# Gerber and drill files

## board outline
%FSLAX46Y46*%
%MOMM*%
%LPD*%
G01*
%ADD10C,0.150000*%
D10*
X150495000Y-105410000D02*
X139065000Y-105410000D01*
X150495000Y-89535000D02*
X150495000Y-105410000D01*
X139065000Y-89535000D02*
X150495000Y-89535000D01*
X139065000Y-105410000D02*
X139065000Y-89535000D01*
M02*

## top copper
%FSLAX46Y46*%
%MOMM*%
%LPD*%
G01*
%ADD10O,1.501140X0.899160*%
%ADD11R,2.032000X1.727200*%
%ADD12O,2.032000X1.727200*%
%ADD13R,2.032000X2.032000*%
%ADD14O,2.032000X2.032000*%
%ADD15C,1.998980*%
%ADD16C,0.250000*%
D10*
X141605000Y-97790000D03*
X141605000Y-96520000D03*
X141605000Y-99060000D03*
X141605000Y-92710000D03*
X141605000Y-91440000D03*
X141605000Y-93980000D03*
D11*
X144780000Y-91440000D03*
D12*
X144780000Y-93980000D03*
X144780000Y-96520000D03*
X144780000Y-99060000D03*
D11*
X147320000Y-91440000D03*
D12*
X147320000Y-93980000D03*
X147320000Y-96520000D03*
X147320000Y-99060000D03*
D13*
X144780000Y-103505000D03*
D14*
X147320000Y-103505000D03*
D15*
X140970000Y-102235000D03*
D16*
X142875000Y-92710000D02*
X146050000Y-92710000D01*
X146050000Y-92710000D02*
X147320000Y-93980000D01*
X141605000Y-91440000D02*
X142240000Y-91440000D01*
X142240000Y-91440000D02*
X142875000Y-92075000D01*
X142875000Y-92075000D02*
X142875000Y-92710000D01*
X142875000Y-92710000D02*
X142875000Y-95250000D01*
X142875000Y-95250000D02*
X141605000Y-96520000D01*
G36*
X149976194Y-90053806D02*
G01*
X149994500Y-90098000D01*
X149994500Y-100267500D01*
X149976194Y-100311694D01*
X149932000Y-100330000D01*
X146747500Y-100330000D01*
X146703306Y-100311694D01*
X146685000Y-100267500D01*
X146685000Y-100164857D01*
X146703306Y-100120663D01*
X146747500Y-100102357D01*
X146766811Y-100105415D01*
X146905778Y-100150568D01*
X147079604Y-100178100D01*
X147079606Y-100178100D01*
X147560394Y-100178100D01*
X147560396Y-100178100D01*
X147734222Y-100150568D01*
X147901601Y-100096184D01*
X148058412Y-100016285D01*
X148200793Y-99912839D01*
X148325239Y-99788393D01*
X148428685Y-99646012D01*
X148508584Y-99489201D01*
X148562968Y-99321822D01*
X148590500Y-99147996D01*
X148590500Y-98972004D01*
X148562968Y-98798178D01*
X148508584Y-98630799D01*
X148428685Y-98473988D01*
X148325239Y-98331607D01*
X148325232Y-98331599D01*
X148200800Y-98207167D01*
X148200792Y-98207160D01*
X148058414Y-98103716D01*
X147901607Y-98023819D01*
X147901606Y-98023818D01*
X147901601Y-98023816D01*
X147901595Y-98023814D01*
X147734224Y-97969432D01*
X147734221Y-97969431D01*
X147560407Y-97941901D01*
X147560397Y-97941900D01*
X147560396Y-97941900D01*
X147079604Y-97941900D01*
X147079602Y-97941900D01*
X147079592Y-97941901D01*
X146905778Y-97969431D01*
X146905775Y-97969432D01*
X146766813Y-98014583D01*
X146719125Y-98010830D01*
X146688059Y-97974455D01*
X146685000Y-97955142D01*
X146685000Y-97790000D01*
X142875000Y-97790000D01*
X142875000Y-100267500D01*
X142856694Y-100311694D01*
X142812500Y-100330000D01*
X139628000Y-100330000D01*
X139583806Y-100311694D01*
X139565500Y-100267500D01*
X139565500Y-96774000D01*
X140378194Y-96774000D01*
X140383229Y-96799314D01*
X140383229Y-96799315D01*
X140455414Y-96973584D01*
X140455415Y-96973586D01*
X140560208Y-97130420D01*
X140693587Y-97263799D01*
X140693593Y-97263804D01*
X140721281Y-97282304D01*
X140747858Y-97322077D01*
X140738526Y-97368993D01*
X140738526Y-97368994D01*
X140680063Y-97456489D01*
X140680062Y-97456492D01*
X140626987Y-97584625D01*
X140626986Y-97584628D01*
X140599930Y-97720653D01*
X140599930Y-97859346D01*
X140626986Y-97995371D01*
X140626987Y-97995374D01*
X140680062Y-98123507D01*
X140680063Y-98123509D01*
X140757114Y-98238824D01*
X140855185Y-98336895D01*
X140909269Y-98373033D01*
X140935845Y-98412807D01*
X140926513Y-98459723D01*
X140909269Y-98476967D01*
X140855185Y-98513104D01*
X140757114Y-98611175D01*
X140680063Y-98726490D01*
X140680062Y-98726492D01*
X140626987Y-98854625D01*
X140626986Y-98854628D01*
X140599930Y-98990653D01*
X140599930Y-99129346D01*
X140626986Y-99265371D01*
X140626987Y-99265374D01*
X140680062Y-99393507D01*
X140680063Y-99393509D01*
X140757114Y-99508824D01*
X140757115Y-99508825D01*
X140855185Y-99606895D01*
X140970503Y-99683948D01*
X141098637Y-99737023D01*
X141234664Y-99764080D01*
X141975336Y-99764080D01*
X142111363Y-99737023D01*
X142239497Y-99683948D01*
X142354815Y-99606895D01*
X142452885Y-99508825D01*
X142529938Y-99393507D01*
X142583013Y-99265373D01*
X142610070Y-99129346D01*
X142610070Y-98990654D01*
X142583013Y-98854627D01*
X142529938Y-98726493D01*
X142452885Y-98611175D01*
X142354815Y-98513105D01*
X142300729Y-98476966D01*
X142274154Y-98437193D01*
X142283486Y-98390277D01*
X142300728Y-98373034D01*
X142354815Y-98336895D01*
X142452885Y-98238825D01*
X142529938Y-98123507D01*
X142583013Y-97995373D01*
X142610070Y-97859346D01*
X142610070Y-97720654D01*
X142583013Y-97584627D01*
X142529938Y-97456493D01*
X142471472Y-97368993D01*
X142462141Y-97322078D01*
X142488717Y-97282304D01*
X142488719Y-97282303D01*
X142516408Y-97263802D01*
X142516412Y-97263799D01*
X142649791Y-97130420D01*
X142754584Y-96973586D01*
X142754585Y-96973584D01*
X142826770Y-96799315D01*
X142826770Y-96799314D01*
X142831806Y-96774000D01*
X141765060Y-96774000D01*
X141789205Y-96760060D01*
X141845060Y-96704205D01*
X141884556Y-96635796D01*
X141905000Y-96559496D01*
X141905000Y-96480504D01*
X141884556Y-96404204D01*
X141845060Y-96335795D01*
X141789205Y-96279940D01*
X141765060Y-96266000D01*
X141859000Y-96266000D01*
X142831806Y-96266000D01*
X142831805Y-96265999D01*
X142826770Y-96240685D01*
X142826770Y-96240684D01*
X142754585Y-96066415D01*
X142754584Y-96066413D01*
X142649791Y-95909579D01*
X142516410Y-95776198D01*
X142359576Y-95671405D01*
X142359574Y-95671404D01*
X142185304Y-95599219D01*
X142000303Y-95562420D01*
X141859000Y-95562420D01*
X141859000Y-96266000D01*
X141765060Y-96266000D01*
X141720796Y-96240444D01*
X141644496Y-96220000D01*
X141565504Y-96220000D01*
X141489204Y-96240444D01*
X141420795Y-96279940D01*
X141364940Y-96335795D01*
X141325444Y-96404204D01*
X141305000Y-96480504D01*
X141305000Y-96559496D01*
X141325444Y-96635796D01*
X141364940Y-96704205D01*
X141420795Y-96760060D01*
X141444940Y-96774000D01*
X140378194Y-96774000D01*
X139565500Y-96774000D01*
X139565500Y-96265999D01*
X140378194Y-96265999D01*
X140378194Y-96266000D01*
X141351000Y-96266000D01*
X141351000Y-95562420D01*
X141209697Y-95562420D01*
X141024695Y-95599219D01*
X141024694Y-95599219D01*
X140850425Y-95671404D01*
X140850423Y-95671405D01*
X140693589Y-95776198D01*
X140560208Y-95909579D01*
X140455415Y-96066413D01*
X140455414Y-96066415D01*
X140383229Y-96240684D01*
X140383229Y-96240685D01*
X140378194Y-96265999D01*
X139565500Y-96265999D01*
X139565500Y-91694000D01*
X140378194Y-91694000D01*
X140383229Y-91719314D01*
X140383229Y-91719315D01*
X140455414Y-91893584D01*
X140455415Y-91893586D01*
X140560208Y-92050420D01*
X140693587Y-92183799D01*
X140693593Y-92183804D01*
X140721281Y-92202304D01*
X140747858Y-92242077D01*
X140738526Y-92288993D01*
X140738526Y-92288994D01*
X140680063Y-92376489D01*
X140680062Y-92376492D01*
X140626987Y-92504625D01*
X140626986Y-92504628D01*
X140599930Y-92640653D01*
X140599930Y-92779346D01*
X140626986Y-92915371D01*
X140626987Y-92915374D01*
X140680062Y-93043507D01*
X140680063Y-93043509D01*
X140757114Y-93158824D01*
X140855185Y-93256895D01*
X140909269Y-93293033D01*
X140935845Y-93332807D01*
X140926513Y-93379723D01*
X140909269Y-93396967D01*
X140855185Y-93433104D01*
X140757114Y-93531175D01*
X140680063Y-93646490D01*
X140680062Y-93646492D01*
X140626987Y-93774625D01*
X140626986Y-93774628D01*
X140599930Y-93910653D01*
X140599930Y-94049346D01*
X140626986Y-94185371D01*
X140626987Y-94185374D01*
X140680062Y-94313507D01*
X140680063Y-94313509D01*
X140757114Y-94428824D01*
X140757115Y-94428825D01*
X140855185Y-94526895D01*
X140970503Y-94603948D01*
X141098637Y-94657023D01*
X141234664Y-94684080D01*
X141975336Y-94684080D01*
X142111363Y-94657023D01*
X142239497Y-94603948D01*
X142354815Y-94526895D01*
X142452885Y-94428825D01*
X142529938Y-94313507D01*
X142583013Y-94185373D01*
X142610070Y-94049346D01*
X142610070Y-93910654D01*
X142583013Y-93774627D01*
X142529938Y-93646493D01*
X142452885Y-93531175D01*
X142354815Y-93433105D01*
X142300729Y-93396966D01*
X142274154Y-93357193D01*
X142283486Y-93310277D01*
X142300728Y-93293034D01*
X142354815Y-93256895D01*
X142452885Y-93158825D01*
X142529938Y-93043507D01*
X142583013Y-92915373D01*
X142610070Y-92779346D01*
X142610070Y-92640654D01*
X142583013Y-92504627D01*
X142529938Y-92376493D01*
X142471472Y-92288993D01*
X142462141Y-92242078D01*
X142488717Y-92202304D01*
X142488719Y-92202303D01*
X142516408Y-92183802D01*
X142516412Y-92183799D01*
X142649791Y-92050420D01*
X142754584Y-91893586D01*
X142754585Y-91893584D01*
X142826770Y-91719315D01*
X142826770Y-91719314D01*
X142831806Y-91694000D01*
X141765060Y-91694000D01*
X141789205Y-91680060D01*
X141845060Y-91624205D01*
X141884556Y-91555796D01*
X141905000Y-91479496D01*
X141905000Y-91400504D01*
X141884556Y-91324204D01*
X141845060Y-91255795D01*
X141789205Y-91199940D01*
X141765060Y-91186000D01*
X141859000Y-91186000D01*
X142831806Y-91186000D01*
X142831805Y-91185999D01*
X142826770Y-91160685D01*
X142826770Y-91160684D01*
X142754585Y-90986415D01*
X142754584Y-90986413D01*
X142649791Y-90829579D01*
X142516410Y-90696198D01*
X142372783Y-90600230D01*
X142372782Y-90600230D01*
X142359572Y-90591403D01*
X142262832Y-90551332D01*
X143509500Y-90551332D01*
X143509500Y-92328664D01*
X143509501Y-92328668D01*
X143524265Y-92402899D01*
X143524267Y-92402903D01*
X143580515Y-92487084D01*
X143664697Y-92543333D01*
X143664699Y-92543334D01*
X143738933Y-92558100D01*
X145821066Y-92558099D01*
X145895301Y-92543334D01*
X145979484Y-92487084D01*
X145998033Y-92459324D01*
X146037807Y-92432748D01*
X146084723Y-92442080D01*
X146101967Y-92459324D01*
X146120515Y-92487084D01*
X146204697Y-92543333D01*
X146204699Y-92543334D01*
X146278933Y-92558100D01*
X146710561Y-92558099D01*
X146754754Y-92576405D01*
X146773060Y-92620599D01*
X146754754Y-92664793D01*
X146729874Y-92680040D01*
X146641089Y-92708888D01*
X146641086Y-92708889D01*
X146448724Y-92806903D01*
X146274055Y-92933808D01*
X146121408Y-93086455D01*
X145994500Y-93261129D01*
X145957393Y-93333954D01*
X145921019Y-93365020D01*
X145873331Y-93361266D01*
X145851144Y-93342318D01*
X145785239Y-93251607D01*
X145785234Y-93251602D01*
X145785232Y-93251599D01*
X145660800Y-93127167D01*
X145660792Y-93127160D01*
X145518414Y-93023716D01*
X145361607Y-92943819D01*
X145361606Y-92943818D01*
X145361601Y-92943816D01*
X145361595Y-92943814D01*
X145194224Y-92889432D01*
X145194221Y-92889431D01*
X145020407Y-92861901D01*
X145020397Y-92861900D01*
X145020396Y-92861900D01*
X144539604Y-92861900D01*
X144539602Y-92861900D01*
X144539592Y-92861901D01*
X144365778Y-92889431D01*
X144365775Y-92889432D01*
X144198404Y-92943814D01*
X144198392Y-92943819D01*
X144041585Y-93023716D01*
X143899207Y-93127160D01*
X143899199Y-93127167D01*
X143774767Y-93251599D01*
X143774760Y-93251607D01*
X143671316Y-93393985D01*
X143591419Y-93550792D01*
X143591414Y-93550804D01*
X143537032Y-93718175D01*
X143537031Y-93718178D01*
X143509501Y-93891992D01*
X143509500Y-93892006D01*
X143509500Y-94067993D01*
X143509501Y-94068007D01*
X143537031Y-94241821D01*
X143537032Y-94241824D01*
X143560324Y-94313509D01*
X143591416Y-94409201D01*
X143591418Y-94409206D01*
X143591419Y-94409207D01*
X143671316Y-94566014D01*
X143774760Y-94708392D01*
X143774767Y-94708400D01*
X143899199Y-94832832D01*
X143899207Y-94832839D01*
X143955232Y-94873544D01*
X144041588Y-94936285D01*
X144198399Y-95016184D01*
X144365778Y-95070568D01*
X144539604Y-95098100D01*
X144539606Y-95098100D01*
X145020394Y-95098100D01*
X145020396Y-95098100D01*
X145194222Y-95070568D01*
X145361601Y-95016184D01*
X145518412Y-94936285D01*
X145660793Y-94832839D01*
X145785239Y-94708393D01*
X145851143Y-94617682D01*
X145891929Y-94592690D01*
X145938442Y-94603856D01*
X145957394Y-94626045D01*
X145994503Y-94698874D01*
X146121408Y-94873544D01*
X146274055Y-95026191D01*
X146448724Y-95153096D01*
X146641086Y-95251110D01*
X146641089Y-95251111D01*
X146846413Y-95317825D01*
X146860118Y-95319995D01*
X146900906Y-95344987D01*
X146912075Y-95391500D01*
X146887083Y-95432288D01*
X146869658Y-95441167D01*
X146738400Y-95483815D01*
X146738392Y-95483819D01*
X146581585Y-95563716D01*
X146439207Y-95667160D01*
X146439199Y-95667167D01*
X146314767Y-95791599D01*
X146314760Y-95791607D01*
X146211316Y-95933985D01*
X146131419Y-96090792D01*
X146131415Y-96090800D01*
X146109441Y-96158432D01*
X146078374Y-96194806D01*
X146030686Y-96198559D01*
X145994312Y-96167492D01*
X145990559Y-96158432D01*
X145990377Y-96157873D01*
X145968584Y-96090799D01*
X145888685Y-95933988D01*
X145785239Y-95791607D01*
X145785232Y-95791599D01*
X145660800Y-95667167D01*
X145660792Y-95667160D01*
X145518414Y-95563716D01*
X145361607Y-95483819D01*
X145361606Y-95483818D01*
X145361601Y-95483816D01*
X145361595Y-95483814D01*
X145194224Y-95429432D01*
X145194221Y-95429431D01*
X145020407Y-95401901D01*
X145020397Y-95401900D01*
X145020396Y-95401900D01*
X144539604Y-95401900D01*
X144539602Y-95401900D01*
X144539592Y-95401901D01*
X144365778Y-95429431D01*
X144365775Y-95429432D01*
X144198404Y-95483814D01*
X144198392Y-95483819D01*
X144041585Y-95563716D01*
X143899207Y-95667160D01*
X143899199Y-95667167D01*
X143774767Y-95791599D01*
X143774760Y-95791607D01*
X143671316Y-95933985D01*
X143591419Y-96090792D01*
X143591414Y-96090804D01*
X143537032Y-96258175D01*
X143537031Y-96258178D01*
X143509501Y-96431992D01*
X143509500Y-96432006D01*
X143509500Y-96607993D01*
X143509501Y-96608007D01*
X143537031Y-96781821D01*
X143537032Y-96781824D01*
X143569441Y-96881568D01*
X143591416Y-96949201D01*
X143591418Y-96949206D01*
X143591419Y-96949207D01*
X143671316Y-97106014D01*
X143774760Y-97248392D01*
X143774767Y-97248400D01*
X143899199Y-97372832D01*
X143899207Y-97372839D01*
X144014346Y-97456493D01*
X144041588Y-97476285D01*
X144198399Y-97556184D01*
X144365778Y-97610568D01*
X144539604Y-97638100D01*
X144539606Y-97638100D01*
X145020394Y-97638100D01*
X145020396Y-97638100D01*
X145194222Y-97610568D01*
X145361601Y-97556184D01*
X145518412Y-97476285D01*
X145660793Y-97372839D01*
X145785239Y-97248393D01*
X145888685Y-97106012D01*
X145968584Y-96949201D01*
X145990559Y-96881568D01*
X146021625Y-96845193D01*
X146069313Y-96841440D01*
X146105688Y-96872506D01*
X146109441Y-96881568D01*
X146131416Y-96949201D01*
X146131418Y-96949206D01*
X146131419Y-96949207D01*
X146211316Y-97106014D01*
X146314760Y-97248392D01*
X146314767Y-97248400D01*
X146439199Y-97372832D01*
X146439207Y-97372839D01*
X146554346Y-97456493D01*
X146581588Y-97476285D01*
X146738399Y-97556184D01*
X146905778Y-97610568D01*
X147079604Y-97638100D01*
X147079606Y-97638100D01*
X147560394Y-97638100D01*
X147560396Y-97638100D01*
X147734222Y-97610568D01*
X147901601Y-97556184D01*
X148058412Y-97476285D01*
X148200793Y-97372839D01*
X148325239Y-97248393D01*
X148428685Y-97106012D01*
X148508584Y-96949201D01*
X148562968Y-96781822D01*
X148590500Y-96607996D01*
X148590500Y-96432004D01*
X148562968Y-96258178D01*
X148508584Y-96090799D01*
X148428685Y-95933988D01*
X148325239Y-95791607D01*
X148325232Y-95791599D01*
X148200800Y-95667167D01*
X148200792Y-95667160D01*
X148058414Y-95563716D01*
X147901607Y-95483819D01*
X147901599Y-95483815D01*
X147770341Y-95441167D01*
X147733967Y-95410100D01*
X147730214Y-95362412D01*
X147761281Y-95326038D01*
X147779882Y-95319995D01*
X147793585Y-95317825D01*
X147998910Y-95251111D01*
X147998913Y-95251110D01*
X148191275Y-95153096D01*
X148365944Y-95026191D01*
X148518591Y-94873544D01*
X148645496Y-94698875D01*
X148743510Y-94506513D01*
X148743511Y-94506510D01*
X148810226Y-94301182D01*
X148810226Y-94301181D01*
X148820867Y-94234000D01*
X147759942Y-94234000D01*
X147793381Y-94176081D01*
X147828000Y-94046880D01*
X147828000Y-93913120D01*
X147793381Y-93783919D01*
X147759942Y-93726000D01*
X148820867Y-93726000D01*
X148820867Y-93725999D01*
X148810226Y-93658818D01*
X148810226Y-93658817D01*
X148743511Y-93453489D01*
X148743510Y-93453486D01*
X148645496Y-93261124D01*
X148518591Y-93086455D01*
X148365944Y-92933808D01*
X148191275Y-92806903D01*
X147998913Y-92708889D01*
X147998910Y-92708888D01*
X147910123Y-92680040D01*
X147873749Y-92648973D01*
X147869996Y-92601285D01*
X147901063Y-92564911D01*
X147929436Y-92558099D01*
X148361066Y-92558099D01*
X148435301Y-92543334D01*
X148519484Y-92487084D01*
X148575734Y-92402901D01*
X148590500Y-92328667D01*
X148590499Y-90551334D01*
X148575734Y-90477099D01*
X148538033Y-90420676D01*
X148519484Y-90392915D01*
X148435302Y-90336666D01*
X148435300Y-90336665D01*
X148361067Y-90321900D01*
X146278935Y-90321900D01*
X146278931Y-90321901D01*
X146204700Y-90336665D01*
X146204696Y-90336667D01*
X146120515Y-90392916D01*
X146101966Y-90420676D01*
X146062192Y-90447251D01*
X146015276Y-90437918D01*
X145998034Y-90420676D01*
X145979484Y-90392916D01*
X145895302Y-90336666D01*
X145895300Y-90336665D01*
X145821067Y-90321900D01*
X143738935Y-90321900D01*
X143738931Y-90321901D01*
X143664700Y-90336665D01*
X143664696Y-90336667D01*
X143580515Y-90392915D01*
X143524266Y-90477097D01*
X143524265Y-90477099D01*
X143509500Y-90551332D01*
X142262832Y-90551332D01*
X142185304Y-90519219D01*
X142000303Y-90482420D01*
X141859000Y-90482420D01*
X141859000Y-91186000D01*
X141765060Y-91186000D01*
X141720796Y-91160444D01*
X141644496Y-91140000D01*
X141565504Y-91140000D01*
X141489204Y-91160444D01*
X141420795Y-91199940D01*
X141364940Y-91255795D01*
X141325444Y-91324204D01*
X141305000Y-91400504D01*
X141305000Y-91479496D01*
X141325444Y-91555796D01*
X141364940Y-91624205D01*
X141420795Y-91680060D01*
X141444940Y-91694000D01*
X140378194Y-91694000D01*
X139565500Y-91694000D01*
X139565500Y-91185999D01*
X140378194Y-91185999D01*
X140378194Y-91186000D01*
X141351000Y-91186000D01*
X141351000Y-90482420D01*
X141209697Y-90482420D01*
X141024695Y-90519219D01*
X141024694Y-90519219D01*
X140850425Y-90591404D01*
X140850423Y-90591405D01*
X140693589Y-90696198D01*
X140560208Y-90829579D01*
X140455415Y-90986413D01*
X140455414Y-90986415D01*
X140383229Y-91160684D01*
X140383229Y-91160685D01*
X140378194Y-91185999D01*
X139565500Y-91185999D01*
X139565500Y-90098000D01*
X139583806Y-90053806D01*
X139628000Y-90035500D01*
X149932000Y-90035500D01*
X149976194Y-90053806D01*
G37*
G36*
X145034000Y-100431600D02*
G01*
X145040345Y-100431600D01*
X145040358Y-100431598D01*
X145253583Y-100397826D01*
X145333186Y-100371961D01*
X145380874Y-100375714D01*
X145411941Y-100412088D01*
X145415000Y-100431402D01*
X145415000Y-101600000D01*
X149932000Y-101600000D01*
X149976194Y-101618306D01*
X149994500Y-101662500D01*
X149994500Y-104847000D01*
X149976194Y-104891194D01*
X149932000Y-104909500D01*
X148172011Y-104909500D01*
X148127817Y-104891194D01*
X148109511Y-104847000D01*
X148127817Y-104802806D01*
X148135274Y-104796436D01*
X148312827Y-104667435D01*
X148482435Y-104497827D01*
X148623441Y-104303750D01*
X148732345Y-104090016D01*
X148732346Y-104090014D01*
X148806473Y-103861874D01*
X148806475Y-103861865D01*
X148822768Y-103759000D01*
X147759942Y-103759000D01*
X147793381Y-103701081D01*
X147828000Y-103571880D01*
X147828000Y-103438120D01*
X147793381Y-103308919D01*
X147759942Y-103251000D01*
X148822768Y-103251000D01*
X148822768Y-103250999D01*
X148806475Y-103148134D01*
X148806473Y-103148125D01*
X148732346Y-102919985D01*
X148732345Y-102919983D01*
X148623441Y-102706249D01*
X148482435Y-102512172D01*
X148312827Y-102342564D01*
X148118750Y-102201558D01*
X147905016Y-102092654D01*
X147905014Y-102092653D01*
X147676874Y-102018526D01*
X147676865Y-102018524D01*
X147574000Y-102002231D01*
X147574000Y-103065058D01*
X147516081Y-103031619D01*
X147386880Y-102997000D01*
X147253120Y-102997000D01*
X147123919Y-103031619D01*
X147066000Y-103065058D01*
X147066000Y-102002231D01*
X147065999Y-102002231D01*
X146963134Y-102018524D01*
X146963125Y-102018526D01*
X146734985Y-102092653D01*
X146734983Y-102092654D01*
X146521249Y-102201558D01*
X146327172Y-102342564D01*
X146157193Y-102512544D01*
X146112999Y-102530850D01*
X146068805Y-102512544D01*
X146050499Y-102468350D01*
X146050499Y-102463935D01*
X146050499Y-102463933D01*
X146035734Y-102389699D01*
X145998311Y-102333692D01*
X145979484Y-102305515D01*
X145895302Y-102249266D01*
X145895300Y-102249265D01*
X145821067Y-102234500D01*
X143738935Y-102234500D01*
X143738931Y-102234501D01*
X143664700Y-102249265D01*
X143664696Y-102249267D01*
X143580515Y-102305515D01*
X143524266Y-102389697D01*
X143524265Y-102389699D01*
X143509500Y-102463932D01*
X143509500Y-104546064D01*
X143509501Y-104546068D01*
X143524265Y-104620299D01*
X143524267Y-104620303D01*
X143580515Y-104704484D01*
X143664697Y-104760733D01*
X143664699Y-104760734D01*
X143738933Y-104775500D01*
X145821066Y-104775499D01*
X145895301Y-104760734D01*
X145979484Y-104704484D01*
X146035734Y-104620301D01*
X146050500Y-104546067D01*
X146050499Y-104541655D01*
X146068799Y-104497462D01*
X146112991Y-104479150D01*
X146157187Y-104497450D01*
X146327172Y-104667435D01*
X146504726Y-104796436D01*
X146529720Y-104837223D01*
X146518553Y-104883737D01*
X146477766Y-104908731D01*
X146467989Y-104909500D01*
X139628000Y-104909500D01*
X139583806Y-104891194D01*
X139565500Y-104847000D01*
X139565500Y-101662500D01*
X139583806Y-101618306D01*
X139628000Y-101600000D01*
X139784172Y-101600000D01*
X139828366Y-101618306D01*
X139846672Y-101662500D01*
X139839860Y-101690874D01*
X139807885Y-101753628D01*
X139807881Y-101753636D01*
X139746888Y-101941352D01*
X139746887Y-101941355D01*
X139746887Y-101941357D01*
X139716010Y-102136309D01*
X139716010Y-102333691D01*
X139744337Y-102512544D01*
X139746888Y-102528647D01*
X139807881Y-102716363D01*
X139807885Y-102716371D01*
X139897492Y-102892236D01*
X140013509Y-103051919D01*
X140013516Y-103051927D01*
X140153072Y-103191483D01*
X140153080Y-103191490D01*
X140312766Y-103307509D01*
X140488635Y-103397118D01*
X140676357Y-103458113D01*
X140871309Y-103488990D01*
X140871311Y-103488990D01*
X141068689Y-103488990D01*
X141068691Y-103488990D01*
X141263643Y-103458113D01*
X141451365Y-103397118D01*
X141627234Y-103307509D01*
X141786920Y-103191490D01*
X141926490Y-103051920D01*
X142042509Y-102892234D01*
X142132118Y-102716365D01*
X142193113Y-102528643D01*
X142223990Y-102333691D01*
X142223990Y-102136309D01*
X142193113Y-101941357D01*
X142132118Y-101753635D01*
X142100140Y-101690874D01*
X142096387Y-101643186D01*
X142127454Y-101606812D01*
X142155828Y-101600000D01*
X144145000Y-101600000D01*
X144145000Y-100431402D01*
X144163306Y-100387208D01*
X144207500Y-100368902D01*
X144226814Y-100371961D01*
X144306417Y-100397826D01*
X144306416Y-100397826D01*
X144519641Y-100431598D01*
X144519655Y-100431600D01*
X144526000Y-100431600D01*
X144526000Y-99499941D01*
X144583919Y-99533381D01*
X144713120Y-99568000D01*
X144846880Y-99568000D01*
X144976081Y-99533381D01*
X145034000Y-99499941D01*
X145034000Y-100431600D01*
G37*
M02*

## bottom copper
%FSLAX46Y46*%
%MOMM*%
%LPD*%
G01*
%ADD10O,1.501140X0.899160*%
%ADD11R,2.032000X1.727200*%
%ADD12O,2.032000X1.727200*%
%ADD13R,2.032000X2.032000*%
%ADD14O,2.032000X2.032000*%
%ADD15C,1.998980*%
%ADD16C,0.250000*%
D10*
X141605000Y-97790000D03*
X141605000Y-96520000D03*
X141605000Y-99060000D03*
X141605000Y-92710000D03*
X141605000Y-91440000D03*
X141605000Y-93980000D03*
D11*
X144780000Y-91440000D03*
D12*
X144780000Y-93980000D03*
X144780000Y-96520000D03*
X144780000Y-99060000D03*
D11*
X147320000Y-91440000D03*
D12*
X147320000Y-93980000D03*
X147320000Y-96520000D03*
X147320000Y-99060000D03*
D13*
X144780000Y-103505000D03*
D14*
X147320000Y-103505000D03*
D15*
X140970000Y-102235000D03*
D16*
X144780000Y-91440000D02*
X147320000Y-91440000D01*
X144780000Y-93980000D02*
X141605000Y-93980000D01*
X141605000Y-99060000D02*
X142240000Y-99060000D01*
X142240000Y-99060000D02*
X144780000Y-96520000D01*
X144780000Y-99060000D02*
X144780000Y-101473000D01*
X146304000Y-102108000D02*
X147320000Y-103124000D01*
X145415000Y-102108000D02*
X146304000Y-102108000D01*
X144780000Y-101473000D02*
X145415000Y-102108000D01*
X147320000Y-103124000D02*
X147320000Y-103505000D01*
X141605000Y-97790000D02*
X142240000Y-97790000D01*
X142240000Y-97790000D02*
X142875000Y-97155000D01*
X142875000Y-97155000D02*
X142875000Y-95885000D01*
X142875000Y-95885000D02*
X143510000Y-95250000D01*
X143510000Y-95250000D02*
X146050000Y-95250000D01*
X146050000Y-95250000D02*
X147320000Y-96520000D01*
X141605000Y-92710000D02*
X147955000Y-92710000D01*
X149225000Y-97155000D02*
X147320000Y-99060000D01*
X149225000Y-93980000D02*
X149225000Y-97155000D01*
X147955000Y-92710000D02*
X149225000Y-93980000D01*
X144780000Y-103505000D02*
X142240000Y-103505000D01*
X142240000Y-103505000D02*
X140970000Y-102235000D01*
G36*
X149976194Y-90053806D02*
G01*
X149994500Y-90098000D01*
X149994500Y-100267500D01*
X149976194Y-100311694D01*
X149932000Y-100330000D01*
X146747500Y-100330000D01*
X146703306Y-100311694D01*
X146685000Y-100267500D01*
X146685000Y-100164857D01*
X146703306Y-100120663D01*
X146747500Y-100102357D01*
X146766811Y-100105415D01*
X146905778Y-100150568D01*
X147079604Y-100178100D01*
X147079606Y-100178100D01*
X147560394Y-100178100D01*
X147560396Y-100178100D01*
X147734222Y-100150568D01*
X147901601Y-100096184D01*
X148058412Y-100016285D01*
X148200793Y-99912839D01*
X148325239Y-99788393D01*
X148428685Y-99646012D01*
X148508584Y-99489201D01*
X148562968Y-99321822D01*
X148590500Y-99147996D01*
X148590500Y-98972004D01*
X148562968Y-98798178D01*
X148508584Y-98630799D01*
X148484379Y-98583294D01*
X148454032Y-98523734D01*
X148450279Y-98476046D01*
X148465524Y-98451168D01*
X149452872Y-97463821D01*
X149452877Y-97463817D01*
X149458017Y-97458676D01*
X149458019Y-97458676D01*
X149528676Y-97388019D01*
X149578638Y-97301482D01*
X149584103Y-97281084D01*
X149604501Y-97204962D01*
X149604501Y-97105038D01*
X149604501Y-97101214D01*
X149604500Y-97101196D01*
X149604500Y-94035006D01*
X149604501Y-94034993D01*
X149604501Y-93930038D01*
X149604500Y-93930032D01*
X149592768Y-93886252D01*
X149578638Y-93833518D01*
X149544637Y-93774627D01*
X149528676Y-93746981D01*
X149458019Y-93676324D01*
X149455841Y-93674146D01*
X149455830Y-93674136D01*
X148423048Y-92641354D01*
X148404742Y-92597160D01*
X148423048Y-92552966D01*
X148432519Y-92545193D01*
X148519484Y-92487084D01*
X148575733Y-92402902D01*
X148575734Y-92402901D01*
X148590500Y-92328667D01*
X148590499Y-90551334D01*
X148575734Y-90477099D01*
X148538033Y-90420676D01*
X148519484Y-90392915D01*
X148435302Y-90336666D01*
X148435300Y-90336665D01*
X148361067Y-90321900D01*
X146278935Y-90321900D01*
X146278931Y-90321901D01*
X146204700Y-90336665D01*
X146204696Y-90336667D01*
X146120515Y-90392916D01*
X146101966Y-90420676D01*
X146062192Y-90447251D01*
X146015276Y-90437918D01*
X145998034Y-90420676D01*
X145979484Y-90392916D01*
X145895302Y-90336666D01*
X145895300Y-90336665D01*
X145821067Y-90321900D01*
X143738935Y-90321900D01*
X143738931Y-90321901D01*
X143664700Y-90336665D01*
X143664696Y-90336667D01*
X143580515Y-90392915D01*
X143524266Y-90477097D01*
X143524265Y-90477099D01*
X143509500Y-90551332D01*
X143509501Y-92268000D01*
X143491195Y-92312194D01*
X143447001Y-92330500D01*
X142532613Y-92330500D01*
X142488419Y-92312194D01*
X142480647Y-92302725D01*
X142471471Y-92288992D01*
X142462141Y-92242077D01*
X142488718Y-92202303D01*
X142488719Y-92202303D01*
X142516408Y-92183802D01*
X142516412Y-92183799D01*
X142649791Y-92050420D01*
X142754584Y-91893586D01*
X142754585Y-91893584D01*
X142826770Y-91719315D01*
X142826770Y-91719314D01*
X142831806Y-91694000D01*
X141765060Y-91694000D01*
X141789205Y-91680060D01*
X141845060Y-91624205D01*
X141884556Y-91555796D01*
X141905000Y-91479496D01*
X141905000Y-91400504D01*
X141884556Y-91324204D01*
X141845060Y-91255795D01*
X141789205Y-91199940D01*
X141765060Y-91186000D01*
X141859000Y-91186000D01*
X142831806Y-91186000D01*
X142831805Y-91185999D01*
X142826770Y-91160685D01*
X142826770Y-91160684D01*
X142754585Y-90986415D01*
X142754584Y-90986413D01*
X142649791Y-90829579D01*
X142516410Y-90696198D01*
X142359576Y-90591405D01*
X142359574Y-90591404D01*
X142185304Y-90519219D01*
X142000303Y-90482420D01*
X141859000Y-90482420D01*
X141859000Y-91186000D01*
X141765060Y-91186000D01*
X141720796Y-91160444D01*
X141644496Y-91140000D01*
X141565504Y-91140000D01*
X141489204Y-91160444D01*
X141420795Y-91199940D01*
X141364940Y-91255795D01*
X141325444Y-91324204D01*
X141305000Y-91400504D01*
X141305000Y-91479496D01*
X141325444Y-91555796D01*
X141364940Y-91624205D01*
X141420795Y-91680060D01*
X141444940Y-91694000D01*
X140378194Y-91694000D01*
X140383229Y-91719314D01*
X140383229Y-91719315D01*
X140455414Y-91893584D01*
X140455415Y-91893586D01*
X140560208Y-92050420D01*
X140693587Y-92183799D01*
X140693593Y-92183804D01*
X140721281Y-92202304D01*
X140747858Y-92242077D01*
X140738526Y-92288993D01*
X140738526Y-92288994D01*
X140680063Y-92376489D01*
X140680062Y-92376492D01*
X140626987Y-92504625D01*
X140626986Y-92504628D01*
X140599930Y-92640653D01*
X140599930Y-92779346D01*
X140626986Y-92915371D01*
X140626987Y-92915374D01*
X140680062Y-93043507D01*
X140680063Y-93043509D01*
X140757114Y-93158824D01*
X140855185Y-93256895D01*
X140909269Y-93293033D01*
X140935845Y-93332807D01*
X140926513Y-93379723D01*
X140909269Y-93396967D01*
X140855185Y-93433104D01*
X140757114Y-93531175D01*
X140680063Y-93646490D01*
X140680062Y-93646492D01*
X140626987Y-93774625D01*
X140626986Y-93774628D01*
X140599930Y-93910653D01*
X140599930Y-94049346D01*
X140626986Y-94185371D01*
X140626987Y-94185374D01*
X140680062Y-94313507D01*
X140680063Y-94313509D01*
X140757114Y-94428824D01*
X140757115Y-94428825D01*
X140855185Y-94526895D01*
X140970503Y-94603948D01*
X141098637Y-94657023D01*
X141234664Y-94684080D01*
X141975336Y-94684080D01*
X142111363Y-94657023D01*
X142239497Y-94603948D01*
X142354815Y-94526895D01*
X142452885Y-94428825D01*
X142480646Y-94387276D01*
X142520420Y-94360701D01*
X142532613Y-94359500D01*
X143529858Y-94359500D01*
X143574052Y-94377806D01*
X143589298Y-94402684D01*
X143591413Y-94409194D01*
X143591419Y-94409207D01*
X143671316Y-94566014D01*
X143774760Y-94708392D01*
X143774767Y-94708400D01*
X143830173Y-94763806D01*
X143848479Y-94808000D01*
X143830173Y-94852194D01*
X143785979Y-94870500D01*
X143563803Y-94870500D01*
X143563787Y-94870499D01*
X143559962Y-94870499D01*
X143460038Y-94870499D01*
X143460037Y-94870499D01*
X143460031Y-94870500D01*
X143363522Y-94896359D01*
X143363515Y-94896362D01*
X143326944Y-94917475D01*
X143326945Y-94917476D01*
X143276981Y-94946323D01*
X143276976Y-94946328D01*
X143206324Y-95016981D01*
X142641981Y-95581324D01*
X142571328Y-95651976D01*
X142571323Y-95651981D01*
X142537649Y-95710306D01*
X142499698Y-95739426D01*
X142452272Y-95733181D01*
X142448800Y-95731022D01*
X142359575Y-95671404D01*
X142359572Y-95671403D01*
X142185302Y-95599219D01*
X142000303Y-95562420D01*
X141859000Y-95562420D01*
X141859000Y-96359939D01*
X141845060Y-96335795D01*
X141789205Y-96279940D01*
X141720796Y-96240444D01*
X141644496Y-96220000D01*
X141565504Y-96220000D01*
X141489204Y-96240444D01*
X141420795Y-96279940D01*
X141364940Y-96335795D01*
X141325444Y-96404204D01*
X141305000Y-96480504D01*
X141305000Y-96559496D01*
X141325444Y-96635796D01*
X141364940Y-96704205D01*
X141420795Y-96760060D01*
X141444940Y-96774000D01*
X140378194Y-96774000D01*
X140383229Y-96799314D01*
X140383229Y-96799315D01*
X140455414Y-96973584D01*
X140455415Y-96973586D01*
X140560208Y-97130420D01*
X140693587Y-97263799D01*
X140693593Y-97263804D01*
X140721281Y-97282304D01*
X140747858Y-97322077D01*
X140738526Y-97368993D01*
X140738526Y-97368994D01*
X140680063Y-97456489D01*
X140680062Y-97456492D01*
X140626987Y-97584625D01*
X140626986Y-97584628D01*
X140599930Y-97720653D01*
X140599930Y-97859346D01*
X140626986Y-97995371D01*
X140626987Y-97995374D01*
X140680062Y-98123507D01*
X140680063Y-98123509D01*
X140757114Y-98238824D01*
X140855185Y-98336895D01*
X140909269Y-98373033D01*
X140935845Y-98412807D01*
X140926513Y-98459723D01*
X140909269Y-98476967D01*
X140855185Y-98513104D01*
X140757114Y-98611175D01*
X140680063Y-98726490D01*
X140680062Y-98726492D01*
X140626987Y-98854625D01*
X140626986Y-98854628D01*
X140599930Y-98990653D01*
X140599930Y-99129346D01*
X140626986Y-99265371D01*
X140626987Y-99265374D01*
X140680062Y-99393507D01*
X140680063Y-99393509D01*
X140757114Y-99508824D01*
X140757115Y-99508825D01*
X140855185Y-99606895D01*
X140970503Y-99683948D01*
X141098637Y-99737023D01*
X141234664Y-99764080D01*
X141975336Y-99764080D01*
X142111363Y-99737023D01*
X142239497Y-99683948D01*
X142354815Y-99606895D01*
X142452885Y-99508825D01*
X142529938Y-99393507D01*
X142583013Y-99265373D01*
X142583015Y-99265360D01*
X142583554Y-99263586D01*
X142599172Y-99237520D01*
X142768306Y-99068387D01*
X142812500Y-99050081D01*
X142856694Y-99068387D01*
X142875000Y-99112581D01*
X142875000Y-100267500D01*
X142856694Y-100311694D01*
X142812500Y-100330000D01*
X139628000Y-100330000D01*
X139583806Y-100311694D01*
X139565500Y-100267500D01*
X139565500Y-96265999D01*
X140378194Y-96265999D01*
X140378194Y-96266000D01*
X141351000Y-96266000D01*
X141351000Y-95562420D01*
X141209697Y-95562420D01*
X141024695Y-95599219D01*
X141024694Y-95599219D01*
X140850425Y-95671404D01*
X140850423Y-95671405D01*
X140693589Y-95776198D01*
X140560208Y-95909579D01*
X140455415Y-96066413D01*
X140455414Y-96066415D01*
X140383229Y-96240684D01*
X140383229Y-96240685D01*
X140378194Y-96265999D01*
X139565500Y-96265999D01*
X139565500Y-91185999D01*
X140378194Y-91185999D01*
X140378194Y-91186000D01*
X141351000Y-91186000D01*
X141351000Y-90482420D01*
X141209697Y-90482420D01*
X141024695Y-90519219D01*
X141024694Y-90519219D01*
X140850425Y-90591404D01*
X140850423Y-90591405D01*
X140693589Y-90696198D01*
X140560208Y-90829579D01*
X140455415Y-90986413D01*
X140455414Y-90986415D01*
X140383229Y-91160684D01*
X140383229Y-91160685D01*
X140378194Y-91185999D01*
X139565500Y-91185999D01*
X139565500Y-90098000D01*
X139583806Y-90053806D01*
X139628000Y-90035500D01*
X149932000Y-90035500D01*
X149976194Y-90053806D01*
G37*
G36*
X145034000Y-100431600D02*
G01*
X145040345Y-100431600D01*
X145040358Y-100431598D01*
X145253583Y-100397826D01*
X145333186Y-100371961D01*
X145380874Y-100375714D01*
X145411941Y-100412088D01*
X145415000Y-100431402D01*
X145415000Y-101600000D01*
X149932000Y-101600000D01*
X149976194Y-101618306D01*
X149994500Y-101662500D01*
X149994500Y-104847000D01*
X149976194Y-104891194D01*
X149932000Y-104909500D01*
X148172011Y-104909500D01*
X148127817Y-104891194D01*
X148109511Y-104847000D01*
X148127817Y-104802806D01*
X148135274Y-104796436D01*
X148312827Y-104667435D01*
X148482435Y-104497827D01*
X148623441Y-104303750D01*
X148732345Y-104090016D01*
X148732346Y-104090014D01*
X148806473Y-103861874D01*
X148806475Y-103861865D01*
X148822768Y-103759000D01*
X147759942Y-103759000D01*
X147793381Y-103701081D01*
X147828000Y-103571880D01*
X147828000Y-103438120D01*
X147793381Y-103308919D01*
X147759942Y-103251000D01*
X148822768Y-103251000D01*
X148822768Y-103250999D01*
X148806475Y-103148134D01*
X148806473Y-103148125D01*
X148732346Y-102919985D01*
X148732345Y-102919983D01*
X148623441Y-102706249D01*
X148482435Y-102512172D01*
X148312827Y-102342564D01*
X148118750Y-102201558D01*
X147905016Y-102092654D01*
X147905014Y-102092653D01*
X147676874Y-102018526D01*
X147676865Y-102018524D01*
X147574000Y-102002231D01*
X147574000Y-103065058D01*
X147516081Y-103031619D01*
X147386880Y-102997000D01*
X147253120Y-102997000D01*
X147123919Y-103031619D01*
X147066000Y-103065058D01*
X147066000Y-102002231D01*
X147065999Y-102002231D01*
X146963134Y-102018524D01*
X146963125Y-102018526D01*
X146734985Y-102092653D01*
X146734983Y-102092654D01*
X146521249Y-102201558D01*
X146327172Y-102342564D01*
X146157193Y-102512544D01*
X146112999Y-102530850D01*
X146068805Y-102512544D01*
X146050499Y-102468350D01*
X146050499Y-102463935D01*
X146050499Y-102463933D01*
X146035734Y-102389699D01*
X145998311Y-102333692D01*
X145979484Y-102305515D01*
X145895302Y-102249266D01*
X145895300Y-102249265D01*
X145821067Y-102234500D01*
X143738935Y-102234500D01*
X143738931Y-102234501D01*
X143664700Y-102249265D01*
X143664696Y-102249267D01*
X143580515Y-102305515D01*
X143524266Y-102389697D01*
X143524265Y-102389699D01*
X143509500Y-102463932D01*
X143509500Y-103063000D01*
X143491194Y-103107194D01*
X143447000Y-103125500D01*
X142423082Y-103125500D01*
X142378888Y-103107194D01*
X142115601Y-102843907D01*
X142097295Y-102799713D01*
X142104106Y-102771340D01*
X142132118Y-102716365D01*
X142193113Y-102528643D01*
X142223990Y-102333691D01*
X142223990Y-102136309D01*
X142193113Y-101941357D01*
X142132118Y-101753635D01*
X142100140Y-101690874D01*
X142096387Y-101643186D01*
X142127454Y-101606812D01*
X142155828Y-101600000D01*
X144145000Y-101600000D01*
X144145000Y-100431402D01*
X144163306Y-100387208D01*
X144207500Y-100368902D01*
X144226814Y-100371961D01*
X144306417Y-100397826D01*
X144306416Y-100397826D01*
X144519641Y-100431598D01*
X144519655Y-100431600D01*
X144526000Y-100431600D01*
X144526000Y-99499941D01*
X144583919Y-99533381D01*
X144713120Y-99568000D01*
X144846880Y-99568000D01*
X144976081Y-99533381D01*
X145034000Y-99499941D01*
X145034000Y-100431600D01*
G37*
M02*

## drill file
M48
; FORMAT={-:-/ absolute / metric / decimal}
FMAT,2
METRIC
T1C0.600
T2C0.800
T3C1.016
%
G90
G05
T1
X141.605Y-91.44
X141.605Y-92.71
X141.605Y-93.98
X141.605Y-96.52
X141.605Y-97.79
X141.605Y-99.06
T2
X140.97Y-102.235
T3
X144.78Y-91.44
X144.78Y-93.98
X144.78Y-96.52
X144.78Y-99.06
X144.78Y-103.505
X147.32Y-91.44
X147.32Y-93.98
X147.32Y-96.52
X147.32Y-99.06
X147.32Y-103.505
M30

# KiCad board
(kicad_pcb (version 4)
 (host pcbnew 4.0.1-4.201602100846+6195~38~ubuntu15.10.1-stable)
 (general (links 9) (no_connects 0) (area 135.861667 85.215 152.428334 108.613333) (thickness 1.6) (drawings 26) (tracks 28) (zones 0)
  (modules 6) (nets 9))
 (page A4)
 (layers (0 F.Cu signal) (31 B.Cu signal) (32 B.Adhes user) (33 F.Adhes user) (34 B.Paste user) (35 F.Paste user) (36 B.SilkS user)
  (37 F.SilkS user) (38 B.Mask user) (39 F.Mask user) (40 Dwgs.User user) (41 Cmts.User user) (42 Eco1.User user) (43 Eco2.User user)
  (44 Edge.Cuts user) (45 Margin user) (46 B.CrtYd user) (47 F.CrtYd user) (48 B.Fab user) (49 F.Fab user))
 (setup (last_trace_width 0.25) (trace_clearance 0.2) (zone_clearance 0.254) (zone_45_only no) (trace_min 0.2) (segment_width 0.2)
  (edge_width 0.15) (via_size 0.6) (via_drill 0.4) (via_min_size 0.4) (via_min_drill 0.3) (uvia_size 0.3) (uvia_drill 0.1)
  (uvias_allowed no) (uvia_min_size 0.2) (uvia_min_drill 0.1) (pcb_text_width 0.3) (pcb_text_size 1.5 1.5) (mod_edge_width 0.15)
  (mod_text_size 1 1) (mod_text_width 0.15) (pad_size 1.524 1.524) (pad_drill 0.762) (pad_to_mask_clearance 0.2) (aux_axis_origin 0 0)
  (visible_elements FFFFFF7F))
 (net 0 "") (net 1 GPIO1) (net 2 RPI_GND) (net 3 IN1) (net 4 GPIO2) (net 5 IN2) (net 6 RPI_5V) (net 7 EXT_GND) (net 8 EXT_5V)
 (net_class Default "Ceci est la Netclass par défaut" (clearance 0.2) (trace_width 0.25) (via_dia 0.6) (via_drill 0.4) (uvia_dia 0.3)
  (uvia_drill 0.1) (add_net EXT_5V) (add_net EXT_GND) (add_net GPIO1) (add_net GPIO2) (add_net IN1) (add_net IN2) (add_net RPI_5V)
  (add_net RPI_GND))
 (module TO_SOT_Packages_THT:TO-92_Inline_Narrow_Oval (layer F.Cu) (at 141.605 99.06 90)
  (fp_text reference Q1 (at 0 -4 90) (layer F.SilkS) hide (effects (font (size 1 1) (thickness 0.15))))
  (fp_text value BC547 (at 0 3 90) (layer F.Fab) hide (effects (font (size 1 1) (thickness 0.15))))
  (pad 2 thru_hole oval (at 1.27 0 270) (size 0.89916 1.50114) (drill 0.6) (layers *.Cu *.Mask F.SilkS) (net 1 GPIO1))
  (pad 3 thru_hole oval (at 2.54 0 270) (size 0.89916 1.50114) (drill 0.6) (layers *.Cu *.Mask F.SilkS) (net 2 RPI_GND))
  (pad 1 thru_hole oval (at 0 0 270) (size 0.89916 1.50114) (drill 0.6) (layers *.Cu *.Mask F.SilkS) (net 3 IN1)))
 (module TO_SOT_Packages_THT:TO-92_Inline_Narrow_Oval (layer F.Cu) (at 141.605 93.98 90)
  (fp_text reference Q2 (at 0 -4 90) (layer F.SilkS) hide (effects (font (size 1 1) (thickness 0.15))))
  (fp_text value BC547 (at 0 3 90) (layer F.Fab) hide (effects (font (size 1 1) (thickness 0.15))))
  (pad 2 thru_hole oval (at 1.27 0 270) (size 0.89916 1.50114) (drill 0.6) (layers *.Cu *.Mask F.SilkS) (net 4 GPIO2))
  (pad 3 thru_hole oval (at 2.54 0 270) (size 0.89916 1.50114) (drill 0.6) (layers *.Cu *.Mask F.SilkS) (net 2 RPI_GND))
  (pad 1 thru_hole oval (at 0 0 270) (size 0.89916 1.50114) (drill 0.6) (layers *.Cu *.Mask F.SilkS) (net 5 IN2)))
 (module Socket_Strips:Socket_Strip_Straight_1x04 (layer B.Cu) (at 144.78 91.44 270)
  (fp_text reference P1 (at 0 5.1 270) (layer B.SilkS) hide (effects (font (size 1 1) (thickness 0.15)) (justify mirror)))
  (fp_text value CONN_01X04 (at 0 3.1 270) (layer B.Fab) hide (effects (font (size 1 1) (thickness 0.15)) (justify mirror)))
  (pad 1 thru_hole rect (at 0 0 270) (size 1.7272 2.032) (drill 1.016) (layers *.Cu *.Mask B.SilkS) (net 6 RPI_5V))
  (pad 2 thru_hole oval (at 2.54 0 270) (size 1.7272 2.032) (drill 1.016) (layers *.Cu *.Mask B.SilkS) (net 5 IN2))
  (pad 3 thru_hole oval (at 5.08 0 270) (size 1.7272 2.032) (drill 1.016) (layers *.Cu *.Mask B.SilkS) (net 3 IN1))
  (pad 4 thru_hole oval (at 7.62 0 270) (size 1.7272 2.032) (drill 1.016) (layers *.Cu *.Mask B.SilkS) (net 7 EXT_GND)))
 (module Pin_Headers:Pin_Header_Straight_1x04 (layer F.Cu) (at 147.32 91.44)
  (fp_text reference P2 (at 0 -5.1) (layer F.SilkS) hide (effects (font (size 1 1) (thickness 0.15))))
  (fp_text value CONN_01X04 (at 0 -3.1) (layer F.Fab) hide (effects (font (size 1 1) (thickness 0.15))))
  (pad 1 thru_hole rect (at 0 0) (size 2.032 1.7272) (drill 1.016) (layers *.Cu *.Mask F.SilkS) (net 6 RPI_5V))
  (pad 2 thru_hole oval (at 0 2.54) (size 2.032 1.7272) (drill 1.016) (layers *.Cu *.Mask F.SilkS) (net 2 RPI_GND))
  (pad 3 thru_hole oval (at 0 5.08) (size 2.032 1.7272) (drill 1.016) (layers *.Cu *.Mask F.SilkS) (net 1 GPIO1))
  (pad 4 thru_hole oval (at 0 7.62) (size 2.032 1.7272) (drill 1.016) (layers *.Cu *.Mask F.SilkS) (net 4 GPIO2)))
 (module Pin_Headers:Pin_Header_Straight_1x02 (layer F.Cu) (at 144.78 103.505 90)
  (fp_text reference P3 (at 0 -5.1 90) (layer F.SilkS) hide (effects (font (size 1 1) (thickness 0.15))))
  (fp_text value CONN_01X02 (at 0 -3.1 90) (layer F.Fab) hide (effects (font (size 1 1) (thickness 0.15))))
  (pad 1 thru_hole rect (at 0 0 90) (size 2.032 2.032) (drill 1.016) (layers *.Cu *.Mask F.SilkS) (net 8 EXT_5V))
  (pad 2 thru_hole oval (at 0 2.54 90) (size 2.032 2.032) (drill 1.016) (layers *.Cu *.Mask F.SilkS) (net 7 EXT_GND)))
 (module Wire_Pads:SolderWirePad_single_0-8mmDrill (layer F.Cu) (at 140.97 102.235)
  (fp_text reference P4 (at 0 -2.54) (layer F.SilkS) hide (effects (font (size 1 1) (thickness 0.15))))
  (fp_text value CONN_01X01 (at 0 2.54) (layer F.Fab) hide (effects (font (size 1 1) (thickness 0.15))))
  (pad 1 thru_hole circle (at 0 0) (size 1.99898 1.99898) (drill 0.8001) (layers *.Cu *.Mask F.SilkS) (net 8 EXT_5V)))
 (gr_line (start 150.495 105.41) (end 139.065 105.41) (angle 90) (layer Edge.Cuts) (width 0.15))
 (gr_line (start 150.495 89.535) (end 150.495 105.41) (angle 90) (layer Edge.Cuts) (width 0.15))
 (gr_line (start 139.065 89.535) (end 150.495 89.535) (angle 90) (layer Edge.Cuts) (width 0.15))
 (gr_line (start 139.065 105.41) (end 139.065 89.535) (angle 90) (layer Edge.Cuts) (width 0.15))
 (segment (start 144.78 91.44) (end 147.32 91.44) (width 0.25) (layer B.Cu) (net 6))
 (segment (start 144.78 93.98) (end 141.605 93.98) (width 0.25) (layer B.Cu) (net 5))
 (segment (start 141.605 99.06) (end 142.24 99.06) (width 0.25) (layer B.Cu) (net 3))
 (segment (start 142.24 99.06) (end 144.78 96.52) (width 0.25) (layer B.Cu) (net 3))
 (segment (start 144.78 99.06) (end 144.78 101.473) (width 0.25) (layer B.Cu) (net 7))
 (segment (start 146.304 102.108) (end 147.32 103.124) (width 0.25) (layer B.Cu) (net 7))
 (segment (start 145.415 102.108) (end 146.304 102.108) (width 0.25) (layer B.Cu) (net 7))
 (segment (start 144.78 101.473) (end 145.415 102.108) (width 0.25) (layer B.Cu) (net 7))
 (segment (start 147.32 103.124) (end 147.32 103.505) (width 0.25) (layer B.Cu) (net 7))
 (segment (start 142.875 92.71) (end 146.05 92.71) (width 0.25) (layer F.Cu) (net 2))
 (segment (start 146.05 92.71) (end 147.32 93.98) (width 0.25) (layer F.Cu) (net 2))
 (segment (start 141.605 91.44) (end 142.24 91.44) (width 0.25) (layer F.Cu) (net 2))
 (segment (start 142.24 91.44) (end 142.875 92.075) (width 0.25) (layer F.Cu) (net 2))
 (segment (start 142.875 92.075) (end 142.875 92.71) (width 0.25) (layer F.Cu) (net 2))
 (segment (start 142.875 92.71) (end 142.875 95.25) (width 0.25) (layer F.Cu) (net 2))
 (segment (start 142.875 95.25) (end 141.605 96.52) (width 0.25) (layer F.Cu) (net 2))
 (segment (start 141.605 97.79) (end 142.24 97.79) (width 0.25) (layer B.Cu) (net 1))
 (segment (start 142.24 97.79) (end 142.875 97.155) (width 0.25) (layer B.Cu) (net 1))
 (segment (start 142.875 97.155) (end 142.875 95.885) (width 0.25) (layer B.Cu) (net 1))
 (segment (start 142.875 95.885) (end 143.51 95.25) (width 0.25) (layer B.Cu) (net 1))
 (segment (start 143.51 95.25) (end 146.05 95.25) (width 0.25) (layer B.Cu) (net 1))
 (segment (start 146.05 95.25) (end 147.32 96.52) (width 0.25) (layer B.Cu) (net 1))
 (segment (start 141.605 92.71) (end 147.955 92.71) (width 0.25) (layer B.Cu) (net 4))
 (segment (start 149.225 97.155) (end 147.32 99.06) (width 0.25) (layer B.Cu) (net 4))
 (segment (start 149.225 93.98) (end 149.225 97.155) (width 0.25) (layer B.Cu) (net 4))
 (segment (start 147.955 92.71) (end 149.225 93.98) (width 0.25) (layer B.Cu) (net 4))
 (segment (start 144.78 103.505) (end 142.24 103.505) (width 0.25) (layer B.Cu) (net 8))
 (segment (start 142.24 103.505) (end 140.97 102.235) (width 0.25) (layer B.Cu) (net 8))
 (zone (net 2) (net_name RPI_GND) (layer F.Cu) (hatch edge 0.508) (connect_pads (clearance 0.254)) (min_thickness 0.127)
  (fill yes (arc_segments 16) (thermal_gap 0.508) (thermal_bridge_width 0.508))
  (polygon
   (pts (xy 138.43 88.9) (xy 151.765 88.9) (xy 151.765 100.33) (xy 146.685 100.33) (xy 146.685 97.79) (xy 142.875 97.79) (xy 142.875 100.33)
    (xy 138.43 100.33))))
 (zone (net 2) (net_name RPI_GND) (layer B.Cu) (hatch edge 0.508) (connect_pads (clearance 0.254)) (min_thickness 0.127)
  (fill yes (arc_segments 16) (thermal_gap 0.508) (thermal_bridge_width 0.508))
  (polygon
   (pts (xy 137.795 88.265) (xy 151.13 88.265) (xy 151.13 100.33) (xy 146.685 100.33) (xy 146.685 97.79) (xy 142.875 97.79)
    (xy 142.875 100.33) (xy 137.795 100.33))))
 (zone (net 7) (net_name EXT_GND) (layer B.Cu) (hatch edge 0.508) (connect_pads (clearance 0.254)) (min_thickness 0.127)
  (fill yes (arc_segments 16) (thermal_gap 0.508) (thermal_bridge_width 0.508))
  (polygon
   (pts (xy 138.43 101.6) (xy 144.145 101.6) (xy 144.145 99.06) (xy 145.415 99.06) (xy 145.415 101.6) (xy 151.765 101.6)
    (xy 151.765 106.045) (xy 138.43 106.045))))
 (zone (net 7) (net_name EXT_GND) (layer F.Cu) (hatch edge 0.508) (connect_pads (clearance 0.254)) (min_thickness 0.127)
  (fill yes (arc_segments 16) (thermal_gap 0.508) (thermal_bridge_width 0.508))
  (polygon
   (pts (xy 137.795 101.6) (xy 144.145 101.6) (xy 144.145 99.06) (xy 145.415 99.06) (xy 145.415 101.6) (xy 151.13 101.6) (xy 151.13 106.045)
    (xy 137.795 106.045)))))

